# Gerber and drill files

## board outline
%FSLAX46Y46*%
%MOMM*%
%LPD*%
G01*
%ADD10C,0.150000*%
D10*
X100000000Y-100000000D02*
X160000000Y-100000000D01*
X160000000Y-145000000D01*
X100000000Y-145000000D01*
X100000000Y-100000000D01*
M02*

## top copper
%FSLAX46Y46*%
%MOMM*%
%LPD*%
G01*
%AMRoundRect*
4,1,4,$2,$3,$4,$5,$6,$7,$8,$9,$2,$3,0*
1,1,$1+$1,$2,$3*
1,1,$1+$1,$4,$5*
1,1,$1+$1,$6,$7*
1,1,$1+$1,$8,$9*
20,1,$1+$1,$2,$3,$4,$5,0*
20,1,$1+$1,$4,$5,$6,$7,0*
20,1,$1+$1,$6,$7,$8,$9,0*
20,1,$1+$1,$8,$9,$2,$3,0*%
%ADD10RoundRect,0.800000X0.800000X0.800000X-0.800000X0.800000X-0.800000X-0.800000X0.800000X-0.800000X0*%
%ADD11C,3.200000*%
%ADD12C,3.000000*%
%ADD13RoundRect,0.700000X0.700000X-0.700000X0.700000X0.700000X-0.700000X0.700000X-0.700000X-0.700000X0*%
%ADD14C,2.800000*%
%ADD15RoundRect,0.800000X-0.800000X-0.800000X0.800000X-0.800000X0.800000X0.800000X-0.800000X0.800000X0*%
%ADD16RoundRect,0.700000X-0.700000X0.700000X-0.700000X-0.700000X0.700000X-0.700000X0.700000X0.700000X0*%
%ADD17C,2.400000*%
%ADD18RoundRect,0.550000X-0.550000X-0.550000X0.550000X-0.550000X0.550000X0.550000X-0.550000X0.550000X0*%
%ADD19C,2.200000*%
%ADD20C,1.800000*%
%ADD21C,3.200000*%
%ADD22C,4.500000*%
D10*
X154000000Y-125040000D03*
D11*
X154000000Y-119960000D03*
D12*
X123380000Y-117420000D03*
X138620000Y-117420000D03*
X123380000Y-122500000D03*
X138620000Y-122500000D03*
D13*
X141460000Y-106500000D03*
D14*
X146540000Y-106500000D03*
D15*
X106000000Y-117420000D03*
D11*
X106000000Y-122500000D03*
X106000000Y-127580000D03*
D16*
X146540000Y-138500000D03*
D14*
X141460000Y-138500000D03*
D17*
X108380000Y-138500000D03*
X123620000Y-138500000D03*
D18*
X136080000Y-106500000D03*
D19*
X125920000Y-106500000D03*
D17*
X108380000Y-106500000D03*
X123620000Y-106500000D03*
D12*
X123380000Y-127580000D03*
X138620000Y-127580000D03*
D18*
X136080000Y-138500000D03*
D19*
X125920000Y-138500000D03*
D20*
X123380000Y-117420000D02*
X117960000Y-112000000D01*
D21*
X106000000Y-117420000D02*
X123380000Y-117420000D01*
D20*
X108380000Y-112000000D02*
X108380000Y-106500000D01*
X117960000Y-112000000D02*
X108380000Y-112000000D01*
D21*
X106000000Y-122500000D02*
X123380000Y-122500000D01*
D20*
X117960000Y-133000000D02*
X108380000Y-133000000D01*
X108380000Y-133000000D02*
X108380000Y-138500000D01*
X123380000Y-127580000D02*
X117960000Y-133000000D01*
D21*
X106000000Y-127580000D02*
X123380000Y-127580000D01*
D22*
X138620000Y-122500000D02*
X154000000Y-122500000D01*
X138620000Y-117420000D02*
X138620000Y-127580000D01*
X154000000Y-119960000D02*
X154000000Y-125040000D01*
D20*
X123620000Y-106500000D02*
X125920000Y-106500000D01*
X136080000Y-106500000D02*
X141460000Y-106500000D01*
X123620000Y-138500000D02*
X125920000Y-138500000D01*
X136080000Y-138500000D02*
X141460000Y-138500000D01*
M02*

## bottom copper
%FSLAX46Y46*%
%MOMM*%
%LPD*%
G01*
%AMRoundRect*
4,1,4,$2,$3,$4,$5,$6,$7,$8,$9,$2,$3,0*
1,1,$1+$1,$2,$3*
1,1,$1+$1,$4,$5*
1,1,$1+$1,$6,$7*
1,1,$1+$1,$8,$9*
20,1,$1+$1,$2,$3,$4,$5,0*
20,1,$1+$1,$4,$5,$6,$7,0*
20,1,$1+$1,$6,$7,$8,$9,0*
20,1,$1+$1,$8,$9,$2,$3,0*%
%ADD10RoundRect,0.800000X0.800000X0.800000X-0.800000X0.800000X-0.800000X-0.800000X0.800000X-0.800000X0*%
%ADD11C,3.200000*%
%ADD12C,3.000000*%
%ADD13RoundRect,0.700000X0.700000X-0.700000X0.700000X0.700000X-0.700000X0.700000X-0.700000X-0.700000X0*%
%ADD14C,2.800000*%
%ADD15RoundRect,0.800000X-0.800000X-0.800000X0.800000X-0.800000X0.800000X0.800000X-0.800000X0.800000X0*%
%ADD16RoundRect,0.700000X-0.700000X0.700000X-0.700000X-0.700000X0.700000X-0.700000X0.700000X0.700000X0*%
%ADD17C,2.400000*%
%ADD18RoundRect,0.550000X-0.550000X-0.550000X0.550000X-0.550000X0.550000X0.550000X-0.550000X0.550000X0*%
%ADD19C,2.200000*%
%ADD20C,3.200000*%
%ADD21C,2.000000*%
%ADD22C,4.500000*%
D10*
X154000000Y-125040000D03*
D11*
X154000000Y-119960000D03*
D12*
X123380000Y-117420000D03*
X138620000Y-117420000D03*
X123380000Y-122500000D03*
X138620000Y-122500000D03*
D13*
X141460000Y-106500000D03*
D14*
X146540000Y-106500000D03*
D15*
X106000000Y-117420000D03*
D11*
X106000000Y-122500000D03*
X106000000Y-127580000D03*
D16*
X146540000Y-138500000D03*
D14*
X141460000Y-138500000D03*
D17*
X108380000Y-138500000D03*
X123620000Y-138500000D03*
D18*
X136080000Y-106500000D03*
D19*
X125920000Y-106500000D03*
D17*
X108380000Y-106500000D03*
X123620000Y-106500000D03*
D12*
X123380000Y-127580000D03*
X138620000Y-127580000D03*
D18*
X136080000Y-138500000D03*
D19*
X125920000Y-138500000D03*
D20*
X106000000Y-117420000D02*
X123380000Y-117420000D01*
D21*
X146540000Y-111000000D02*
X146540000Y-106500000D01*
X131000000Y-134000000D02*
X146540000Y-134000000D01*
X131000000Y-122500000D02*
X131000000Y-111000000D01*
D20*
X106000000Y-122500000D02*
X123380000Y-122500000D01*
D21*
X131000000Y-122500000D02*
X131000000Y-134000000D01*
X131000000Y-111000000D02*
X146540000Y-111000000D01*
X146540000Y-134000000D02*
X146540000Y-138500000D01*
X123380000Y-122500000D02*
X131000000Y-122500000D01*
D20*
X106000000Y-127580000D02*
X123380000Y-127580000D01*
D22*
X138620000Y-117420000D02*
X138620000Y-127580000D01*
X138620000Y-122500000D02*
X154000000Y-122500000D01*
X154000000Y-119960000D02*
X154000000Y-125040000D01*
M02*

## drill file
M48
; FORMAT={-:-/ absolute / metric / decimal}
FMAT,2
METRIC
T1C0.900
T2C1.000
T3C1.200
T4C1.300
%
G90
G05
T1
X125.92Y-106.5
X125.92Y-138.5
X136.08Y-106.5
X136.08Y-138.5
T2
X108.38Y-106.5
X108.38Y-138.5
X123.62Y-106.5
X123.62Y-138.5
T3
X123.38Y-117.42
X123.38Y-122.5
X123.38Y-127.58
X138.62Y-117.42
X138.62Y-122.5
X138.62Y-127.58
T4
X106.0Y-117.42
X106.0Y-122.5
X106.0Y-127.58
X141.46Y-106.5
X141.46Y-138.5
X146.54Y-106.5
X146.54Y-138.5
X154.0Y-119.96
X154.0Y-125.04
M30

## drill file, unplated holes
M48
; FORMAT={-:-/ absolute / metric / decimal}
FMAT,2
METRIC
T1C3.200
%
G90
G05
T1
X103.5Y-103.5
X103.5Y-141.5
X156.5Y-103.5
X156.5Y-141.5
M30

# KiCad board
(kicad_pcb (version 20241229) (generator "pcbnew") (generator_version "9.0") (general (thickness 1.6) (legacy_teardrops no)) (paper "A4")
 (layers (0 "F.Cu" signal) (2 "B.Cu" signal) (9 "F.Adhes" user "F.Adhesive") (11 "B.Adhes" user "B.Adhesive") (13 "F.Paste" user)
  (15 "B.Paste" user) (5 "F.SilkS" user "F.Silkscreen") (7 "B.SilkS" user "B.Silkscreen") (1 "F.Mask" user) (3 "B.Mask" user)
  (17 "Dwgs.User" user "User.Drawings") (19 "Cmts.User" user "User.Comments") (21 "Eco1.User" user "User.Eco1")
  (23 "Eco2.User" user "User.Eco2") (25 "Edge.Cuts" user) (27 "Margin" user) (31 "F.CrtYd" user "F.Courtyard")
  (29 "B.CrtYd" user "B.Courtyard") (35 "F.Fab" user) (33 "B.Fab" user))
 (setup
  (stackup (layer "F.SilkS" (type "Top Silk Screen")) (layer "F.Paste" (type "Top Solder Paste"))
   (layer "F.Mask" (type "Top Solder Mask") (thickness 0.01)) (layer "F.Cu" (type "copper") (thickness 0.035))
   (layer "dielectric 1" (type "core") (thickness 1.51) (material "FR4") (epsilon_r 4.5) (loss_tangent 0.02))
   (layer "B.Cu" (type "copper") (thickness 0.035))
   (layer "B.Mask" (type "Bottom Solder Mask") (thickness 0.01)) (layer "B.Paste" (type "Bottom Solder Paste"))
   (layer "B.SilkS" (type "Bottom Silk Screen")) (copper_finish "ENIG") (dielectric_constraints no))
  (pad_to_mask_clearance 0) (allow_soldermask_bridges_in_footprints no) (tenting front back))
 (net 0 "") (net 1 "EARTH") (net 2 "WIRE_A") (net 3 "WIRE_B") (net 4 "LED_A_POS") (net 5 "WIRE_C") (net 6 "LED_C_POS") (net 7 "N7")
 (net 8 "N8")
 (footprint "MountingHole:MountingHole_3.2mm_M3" (layer "F.Cu") (at 156.5 103.5)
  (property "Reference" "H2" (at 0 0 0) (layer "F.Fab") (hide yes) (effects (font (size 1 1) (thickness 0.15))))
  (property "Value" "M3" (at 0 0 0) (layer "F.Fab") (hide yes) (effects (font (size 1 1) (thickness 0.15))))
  (pad "" np_thru_hole circle (at 0 0) (size 3.2 3.2) (drill 3.2) (layers "*.Cu" "*.Mask")))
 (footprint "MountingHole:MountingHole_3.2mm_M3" (layer "F.Cu") (at 156.5 141.5)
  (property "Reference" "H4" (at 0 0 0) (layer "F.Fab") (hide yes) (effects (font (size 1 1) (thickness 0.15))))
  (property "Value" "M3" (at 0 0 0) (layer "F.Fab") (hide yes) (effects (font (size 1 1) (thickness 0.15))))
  (pad "" np_thru_hole circle (at 0 0) (size 3.2 3.2) (drill 3.2) (layers "*.Cu" "*.Mask")))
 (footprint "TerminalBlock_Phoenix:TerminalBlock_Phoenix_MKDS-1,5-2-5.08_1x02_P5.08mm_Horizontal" (layer "F.Cu") (at 154 122.5 180)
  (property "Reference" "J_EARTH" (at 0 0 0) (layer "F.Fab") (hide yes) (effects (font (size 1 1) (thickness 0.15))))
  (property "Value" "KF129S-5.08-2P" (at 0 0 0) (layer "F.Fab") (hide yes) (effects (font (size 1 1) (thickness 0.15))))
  (pad "1" thru_hole roundrect (at 0 -2.54 180) (size 3.2 3.2) (drill 1.3) (layers "*.Cu" "*.Mask") (remove_unused_layers no)
   (roundrect_rratio 0.25) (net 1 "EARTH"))
  (pad "2" thru_hole circle (at 0 2.54 180) (size 3.2 3.2) (drill 1.3) (layers "*.Cu" "*.Mask") (remove_unused_layers no) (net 1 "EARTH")))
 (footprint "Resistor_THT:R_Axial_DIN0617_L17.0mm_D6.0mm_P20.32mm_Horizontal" (layer "F.Cu") (at 131 117.42)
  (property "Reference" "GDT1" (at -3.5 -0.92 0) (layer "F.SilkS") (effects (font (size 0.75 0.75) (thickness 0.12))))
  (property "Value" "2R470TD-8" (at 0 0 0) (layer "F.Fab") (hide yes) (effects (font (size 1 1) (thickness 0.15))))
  (pad "1" thru_hole circle (at -7.62 0) (size 3 3) (drill 1.2) (layers "*.Cu" "*.Mask") (remove_unused_layers no) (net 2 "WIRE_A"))
  (pad "2" thru_hole circle (at 7.62 0) (size 3 3) (drill 1.2) (layers "*.Cu" "*.Mask") (remove_unused_layers no) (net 1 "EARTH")))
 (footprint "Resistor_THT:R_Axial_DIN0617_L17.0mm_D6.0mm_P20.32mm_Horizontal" (layer "F.Cu") (at 131 122.5)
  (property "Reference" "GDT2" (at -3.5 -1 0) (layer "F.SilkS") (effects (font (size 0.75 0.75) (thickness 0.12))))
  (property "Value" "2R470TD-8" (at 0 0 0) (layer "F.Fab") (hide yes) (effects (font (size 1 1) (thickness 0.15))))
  (pad "1" thru_hole circle (at -7.62 0) (size 3 3) (drill 1.2) (layers "*.Cu" "*.Mask") (remove_unused_layers no) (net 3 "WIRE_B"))
  (pad "2" thru_hole circle (at 7.62 0) (size 3 3) (drill 1.2) (layers "*.Cu" "*.Mask") (remove_unused_layers no) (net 1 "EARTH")))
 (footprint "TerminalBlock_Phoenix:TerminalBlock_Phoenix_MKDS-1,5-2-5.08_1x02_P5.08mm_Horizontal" (layer "F.Cu") (at 144 106.5 90)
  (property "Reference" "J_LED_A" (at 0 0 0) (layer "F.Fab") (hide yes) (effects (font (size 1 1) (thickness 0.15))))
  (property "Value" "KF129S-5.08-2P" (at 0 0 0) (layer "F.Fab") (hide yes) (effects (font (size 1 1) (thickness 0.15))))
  (pad "1" thru_hole roundrect (at 0 -2.54 90) (size 2.8 2.8) (drill 1.3) (layers "*.Cu" "*.Mask") (remove_unused_layers no)
   (roundrect_rratio 0.25) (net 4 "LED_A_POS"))
  (pad "2" thru_hole circle (at 0 2.54 90) (size 2.8 2.8) (drill 1.3) (layers "*.Cu" "*.Mask") (remove_unused_layers no) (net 3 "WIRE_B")))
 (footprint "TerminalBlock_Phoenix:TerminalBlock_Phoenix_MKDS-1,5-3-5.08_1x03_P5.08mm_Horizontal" (layer "F.Cu") (at 106 122.5)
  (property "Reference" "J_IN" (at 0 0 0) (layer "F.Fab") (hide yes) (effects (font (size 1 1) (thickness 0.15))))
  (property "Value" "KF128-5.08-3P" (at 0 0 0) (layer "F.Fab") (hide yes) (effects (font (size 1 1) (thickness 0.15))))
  (pad "1" thru_hole roundrect (at 0 -5.08) (size 3.2 3.2) (drill 1.3) (layers "*.Cu" "*.Mask") (remove_unused_layers no)
   (roundrect_rratio 0.25) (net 2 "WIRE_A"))
  (pad "2" thru_hole circle (at 0 0) (size 3.2 3.2) (drill 1.3) (layers "*.Cu" "*.Mask") (remove_unused_layers no) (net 3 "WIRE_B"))
  (pad "3" thru_hole circle (at 0 5.08) (size 3.2 3.2) (drill 1.3) (layers "*.Cu" "*.Mask") (remove_unused_layers no) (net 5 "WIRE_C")))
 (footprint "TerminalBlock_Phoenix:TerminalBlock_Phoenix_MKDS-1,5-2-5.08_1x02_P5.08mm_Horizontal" (layer "F.Cu") (at 144 138.5 -90)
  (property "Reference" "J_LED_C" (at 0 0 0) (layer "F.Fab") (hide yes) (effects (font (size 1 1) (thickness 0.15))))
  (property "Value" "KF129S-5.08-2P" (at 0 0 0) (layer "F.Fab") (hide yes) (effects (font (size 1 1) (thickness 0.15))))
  (pad "1" thru_hole roundrect (at 0 -2.54 270) (size 2.8 2.8) (drill 1.3) (layers "*.Cu" "*.Mask") (remove_unused_layers no)
   (roundrect_rratio 0.25) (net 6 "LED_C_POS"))
  (pad "2" thru_hole circle (at 0 2.54 270) (size 2.8 2.8) (drill 1.3) (layers "*.Cu" "*.Mask") (remove_unused_layers no) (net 3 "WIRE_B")))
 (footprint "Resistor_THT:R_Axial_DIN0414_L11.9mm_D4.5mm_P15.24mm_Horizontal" (layer "F.Cu") (at 116 138.5)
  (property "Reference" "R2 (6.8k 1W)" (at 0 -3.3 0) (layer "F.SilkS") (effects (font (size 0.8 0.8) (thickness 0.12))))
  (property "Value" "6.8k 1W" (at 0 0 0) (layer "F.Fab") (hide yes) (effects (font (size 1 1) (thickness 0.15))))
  (pad "1" thru_hole circle (at -7.62 0) (size 2.4 2.4) (drill 1) (layers "*.Cu" "*.Mask") (remove_unused_layers no) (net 5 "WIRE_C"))
  (pad "2" thru_hole circle (at 7.62 0) (size 2.4 2.4) (drill 1) (layers "*.Cu" "*.Mask") (remove_unused_layers no) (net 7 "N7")))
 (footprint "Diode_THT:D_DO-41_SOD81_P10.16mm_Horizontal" (layer "F.Cu") (at 131 106.5)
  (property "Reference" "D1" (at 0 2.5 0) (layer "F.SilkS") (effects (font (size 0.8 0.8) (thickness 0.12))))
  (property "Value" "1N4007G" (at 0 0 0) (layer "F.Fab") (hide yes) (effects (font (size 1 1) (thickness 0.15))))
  (pad "1" thru_hole roundrect (at 5.08 0) (size 2.2 2.2) (drill 0.9) (layers "*.Cu" "*.Mask") (remove_unused_layers no)
   (roundrect_rratio 0.25) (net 4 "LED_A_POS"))
  (pad "2" thru_hole circle (at -5.08 0) (size 2.2 2.2) (drill 0.9) (layers "*.Cu" "*.Mask") (remove_unused_layers no) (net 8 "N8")))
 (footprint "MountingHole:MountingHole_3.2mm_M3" (layer "F.Cu") (at 103.5 141.5)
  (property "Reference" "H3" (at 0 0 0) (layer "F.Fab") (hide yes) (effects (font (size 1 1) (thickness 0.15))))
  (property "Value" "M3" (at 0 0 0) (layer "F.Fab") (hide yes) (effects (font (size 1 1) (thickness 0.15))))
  (pad "" np_thru_hole circle (at 0 0) (size 3.2 3.2) (drill 3.2) (layers "*.Cu" "*.Mask")))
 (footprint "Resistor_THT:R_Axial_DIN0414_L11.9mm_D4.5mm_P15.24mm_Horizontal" (layer "F.Cu") (at 116 106.5)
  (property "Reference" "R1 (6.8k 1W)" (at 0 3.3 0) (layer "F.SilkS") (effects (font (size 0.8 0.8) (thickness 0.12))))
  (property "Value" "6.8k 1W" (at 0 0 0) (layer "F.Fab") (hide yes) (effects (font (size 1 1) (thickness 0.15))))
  (pad "1" thru_hole circle (at -7.62 0) (size 2.4 2.4) (drill 1) (layers "*.Cu" "*.Mask") (remove_unused_layers no) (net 2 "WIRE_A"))
  (pad "2" thru_hole circle (at 7.62 0) (size 2.4 2.4) (drill 1) (layers "*.Cu" "*.Mask") (remove_unused_layers no) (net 8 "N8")))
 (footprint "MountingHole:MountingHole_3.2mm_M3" (layer "F.Cu") (at 103.5 103.5)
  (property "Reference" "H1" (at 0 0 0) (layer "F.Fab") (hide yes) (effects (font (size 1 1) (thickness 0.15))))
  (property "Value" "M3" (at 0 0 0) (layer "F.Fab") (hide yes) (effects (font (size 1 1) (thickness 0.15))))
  (pad "" np_thru_hole circle (at 0 0) (size 3.2 3.2) (drill 3.2) (layers "*.Cu" "*.Mask")))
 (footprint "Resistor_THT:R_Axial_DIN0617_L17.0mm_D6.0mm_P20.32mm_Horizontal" (layer "F.Cu") (at 131 127.58)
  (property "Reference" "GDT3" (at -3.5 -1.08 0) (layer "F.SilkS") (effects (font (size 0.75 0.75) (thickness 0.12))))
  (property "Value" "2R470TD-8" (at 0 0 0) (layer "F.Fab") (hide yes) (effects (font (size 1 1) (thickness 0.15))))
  (pad "1" thru_hole circle (at -7.62 0) (size 3 3) (drill 1.2) (layers "*.Cu" "*.Mask") (remove_unused_layers no) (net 5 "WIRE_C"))
  (pad "2" thru_hole circle (at 7.62 0) (size 3 3) (drill 1.2) (layers "*.Cu" "*.Mask") (remove_unused_layers no) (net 1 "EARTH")))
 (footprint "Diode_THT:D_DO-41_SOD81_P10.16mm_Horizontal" (layer "F.Cu") (at 131 138.5)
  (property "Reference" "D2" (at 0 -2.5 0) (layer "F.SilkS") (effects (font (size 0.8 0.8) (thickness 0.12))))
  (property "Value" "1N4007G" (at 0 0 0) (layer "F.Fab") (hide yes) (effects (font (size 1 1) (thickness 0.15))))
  (pad "1" thru_hole roundrect (at 5.08 0) (size 2.2 2.2) (drill 0.9) (layers "*.Cu" "*.Mask") (remove_unused_layers no)
   (roundrect_rratio 0.25) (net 6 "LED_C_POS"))
  (pad "2" thru_hole circle (at -5.08 0) (size 2.2 2.2) (drill 0.9) (layers "*.Cu" "*.Mask") (remove_unused_layers no) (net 7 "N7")))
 (gr_rect (start 100 100) (end 160 145) (stroke (width 0.15) (type solid)) (fill no) (layer "Edge.Cuts"))
 (segment (start 123.38 117.42) (end 117.96 112) (width 1.8) (layer "F.Cu") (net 2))
 (segment (start 106 117.42) (end 123.38 117.42) (width 3.2) (layer "F.Cu") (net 2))
 (segment (start 108.38 112) (end 108.38 106.5) (width 1.8) (layer "F.Cu") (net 2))
 (segment (start 117.96 112) (end 108.38 112) (width 1.8) (layer "F.Cu") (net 2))
 (segment (start 106 117.42) (end 123.38 117.42) (width 3.2) (layer "B.Cu") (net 2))
 (segment (start 106 122.5) (end 123.38 122.5) (width 3.2) (layer "F.Cu") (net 3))
 (segment (start 146.54 111) (end 146.54 106.5) (width 2) (layer "B.Cu") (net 3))
 (segment (start 131 134) (end 146.54 134) (width 2) (layer "B.Cu") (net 3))
 (segment (start 131 122.5) (end 131 111) (width 2) (layer "B.Cu") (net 3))
 (segment (start 106 122.5) (end 123.38 122.5) (width 3.2) (layer "B.Cu") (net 3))
 (segment (start 131 122.5) (end 131 134) (width 2) (layer "B.Cu") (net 3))
 (segment (start 131 111) (end 146.54 111) (width 2) (layer "B.Cu") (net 3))
 (segment (start 146.54 134) (end 146.54 138.5) (width 2) (layer "B.Cu") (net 3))
 (segment (start 123.38 122.5) (end 131 122.5) (width 2) (layer "B.Cu") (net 3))
 (segment (start 117.96 133) (end 108.38 133) (width 1.8) (layer "F.Cu") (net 5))
 (segment (start 108.38 133) (end 108.38 138.5) (width 1.8) (layer "F.Cu") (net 5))
 (segment (start 123.38 127.58) (end 117.96 133) (width 1.8) (layer "F.Cu") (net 5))
 (segment (start 106 127.58) (end 123.38 127.58) (width 3.2) (layer "F.Cu") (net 5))
 (segment (start 106 127.58) (end 123.38 127.58) (width 3.2) (layer "B.Cu") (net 5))
 (segment (start 138.62 122.5) (end 154 122.5) (width 4.5) (layer "F.Cu") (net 1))
 (segment (start 138.62 117.42) (end 138.62 127.58) (width 4.5) (layer "F.Cu") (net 1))
 (segment (start 154 119.96) (end 154 125.04) (width 4.5) (layer "F.Cu") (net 1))
 (segment (start 138.62 117.42) (end 138.62 127.58) (width 4.5) (layer "B.Cu") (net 1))
 (segment (start 138.62 122.5) (end 154 122.5) (width 4.5) (layer "B.Cu") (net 1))
 (segment (start 154 119.96) (end 154 125.04) (width 4.5) (layer "B.Cu") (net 1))
 (segment (start 123.62 106.5) (end 125.92 106.5) (width 1.8) (layer "F.Cu") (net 8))
 (segment (start 136.08 106.5) (end 141.46 106.5) (width 1.8) (layer "F.Cu") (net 4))
 (segment (start 123.62 138.5) (end 125.92 138.5) (width 1.8) (layer "F.Cu") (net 7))
 (segment (start 136.08 138.5) (end 141.46 138.5) (width 1.8) (layer "F.Cu") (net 6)))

